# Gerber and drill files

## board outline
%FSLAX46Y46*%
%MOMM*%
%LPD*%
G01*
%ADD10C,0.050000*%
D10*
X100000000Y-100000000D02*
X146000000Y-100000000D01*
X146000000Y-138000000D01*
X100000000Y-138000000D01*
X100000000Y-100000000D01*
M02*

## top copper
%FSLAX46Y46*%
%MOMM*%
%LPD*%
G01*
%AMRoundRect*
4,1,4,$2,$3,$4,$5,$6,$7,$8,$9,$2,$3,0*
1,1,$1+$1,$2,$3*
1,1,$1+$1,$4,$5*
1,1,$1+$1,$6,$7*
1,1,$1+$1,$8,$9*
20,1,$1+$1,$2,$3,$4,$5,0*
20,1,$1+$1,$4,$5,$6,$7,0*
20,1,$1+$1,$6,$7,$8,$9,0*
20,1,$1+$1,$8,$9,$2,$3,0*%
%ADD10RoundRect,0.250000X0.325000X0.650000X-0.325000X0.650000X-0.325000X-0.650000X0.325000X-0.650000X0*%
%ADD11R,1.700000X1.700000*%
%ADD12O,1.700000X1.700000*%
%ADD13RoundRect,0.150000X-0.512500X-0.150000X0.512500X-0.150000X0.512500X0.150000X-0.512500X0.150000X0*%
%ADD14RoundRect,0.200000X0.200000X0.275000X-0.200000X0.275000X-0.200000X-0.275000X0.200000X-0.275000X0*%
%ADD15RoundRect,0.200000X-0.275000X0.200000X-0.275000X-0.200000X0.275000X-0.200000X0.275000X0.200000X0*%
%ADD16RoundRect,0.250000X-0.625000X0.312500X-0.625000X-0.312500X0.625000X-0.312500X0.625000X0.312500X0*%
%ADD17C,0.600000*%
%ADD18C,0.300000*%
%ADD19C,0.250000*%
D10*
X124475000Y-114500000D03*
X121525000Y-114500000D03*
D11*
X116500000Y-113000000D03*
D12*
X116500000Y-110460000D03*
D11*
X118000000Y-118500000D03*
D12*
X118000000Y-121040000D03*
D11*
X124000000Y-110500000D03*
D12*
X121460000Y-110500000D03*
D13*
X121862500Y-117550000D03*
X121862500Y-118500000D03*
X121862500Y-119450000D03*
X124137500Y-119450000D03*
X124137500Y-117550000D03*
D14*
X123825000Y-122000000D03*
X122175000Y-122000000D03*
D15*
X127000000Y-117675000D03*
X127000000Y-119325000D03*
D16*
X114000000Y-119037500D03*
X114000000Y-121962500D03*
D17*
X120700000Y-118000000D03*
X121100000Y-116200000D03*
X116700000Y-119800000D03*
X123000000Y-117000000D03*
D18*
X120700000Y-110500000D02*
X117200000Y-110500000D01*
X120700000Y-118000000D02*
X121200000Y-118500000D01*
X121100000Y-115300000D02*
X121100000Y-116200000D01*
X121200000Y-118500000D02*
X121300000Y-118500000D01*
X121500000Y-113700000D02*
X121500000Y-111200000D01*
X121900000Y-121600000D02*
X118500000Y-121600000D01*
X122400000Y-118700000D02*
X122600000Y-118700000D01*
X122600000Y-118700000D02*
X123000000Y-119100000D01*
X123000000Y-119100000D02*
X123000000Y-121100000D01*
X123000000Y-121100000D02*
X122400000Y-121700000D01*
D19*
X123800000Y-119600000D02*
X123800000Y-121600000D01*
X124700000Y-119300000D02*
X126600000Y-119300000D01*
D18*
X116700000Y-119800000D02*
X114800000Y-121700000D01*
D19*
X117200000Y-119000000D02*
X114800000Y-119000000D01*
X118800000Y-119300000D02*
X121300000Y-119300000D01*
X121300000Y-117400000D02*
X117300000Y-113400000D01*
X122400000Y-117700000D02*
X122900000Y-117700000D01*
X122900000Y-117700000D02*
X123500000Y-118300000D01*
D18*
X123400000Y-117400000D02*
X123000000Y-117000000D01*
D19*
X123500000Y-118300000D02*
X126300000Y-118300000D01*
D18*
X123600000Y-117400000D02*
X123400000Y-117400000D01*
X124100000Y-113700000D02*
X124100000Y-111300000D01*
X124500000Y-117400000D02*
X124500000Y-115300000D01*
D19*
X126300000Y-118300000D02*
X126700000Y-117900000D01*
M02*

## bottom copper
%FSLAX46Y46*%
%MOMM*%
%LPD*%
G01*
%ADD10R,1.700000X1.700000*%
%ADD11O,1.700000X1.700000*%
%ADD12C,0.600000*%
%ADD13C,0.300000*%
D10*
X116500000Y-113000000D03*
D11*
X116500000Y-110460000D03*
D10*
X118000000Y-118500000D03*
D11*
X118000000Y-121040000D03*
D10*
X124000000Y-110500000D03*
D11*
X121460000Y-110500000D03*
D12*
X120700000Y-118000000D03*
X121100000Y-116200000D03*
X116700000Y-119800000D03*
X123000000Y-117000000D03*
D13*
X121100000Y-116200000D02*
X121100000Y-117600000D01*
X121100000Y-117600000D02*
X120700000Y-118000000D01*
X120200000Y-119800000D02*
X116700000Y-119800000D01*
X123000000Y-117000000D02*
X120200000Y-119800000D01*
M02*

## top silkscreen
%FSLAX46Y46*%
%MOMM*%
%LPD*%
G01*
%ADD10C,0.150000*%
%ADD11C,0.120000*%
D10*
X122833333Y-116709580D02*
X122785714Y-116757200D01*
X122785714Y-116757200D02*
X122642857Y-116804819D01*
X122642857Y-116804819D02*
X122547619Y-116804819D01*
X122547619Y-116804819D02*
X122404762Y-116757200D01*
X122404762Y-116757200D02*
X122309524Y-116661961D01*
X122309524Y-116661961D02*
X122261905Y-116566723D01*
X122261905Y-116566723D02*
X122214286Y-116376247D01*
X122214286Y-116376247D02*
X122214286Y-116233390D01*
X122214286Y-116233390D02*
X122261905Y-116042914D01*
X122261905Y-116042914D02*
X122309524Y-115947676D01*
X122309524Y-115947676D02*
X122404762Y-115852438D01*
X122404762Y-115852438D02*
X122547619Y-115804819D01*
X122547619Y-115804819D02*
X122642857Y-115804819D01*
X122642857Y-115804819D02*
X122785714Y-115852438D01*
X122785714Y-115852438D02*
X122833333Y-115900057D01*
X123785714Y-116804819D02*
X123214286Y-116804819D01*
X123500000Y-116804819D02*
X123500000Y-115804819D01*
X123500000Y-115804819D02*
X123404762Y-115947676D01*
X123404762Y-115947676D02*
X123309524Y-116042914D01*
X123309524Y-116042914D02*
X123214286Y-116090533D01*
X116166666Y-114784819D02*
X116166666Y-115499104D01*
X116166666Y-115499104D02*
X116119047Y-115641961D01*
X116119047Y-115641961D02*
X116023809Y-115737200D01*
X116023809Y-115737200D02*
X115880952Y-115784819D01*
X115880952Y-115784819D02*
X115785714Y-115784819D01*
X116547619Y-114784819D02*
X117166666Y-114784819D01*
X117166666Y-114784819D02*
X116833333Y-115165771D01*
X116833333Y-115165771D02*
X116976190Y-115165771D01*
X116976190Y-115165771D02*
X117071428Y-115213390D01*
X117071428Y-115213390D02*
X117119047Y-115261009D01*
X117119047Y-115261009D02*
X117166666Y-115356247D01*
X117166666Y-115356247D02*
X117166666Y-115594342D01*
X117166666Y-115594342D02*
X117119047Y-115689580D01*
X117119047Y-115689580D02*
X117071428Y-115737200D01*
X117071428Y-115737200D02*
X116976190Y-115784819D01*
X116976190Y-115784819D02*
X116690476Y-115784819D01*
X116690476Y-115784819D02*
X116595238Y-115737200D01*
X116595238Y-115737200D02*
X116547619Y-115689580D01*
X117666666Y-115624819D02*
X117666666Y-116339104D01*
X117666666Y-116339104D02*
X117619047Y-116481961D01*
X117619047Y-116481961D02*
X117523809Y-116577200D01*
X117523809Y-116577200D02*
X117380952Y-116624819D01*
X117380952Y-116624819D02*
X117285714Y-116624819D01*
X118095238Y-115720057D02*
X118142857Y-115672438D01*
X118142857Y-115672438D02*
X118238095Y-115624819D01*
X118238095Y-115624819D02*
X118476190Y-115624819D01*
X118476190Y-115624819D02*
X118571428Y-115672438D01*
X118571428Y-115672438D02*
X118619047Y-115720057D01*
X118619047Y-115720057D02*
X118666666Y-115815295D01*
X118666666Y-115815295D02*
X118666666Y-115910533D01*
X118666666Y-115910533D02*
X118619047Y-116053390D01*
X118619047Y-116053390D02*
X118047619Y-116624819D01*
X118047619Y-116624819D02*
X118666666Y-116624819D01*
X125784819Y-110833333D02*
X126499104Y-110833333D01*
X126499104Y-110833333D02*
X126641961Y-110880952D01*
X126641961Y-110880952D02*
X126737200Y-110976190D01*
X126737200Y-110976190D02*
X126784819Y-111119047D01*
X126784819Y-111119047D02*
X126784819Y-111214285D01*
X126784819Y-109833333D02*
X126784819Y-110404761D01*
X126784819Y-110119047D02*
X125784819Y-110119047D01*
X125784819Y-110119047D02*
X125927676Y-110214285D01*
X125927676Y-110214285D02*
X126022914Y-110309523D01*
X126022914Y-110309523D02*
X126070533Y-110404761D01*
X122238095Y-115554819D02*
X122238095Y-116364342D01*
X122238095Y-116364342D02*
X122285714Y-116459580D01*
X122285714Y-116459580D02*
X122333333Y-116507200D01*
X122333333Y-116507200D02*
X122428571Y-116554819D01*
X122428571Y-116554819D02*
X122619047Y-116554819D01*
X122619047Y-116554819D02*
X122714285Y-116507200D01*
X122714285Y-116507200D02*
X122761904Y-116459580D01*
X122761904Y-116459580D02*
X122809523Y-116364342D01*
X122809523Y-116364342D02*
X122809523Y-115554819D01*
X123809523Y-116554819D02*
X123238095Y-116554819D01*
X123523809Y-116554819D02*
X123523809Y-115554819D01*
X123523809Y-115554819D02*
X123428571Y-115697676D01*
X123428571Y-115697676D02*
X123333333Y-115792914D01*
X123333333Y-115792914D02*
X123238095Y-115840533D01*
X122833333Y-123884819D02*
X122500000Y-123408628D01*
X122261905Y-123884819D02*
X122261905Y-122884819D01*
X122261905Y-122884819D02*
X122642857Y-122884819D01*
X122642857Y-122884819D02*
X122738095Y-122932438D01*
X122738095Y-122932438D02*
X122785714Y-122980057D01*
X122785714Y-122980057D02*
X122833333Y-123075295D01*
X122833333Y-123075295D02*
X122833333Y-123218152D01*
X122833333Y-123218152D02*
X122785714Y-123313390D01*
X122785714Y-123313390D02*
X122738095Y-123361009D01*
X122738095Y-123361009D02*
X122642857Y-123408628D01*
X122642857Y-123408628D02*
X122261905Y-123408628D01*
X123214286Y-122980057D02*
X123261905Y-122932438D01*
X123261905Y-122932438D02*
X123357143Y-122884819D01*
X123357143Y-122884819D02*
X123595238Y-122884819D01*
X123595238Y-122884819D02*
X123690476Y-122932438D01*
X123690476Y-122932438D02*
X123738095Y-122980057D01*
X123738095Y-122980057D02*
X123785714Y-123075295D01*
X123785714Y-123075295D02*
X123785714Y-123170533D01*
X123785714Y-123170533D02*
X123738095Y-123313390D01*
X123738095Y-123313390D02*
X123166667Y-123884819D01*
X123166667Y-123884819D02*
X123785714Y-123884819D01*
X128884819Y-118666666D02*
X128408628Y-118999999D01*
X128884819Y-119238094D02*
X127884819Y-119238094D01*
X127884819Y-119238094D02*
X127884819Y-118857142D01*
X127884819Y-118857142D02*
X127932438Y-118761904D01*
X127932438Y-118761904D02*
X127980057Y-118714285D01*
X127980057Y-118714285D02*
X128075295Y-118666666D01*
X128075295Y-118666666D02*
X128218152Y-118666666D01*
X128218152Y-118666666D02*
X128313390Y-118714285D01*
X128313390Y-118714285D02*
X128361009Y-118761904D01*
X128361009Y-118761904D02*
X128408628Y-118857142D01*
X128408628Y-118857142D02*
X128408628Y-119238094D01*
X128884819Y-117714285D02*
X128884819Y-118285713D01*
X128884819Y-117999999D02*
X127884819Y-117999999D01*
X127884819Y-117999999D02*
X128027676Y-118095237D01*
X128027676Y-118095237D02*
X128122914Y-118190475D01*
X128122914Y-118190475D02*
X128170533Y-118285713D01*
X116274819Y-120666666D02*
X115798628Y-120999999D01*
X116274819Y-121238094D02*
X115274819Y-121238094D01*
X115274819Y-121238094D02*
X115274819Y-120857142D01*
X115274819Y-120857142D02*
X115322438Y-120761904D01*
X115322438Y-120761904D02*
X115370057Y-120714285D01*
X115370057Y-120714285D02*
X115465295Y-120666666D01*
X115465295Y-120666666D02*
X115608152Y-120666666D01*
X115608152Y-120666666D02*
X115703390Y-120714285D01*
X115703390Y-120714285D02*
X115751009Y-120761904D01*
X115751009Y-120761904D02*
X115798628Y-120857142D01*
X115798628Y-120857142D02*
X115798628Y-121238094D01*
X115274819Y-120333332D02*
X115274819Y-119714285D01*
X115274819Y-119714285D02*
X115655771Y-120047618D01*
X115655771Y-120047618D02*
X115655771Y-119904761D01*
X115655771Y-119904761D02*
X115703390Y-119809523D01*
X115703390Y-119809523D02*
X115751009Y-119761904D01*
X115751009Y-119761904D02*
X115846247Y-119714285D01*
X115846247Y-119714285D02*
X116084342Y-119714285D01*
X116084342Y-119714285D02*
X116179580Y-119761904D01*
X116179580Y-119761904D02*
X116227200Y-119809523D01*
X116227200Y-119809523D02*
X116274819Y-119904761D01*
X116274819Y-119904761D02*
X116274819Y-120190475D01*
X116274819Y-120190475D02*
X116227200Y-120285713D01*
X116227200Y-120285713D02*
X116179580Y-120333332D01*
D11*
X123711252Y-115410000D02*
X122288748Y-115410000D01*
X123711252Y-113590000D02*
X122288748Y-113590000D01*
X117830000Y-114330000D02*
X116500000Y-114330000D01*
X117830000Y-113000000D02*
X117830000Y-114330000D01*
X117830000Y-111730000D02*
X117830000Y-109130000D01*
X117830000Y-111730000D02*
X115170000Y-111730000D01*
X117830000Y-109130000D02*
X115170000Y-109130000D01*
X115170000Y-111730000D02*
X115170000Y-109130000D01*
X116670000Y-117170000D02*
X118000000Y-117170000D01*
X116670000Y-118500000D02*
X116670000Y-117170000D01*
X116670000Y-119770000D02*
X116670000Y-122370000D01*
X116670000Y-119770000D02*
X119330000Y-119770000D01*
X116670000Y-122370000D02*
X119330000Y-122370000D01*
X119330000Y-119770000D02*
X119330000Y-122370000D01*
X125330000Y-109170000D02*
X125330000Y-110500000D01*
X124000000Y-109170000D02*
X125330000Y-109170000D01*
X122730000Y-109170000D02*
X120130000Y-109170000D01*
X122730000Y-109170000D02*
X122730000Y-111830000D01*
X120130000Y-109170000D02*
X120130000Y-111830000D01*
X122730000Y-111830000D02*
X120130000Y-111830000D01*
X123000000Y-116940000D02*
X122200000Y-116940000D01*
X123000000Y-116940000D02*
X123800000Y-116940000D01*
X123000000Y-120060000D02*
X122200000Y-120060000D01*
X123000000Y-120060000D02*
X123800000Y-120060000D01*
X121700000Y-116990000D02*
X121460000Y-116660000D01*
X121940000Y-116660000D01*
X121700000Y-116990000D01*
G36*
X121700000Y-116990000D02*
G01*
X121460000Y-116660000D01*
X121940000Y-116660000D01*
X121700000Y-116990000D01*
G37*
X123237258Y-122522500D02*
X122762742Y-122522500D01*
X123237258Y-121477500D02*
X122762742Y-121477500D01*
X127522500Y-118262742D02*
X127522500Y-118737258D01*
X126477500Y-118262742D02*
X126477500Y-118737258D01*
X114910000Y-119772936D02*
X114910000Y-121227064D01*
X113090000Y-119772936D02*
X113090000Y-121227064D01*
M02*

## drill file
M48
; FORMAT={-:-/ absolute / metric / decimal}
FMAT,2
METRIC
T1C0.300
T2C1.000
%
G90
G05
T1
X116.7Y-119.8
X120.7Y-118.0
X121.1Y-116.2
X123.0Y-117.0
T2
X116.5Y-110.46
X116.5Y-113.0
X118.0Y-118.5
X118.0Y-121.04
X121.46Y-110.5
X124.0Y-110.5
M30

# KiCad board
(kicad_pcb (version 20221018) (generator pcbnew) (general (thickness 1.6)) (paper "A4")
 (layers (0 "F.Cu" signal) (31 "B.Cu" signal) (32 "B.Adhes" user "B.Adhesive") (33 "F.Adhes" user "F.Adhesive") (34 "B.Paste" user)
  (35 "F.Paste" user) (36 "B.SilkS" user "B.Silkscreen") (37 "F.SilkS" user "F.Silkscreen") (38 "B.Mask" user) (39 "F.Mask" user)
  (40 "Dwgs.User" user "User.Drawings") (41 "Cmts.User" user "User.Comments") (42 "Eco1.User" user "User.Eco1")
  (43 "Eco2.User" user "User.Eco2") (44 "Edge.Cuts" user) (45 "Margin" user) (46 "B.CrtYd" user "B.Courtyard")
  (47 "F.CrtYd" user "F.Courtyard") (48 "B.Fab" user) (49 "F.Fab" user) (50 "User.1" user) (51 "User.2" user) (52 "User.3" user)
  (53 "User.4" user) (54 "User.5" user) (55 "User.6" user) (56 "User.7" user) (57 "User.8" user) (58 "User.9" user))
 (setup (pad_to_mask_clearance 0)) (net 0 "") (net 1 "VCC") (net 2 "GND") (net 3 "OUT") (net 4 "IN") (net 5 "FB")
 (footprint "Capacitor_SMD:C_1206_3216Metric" (layer "F.Cu") (at 123 114.5 180)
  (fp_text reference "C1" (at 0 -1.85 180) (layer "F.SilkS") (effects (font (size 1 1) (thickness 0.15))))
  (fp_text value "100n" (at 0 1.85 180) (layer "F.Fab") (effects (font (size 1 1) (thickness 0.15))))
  (fp_line (start -0.711252 -0.91) (end 0.711252 -0.91) (stroke (width 0.12) (type solid)) (layer "F.SilkS"))
  (fp_line (start -0.711252 0.91) (end 0.711252 0.91) (stroke (width 0.12) (type solid)) (layer "F.SilkS"))
  (pad "1" smd roundrect (at -1.475 0 180) (size 1.15 1.8) (layers "F.Cu" "F.Paste" "F.Mask") (roundrect_rratio 0.217391) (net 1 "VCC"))
  (pad "2" smd roundrect (at 1.475 0 180) (size 1.15 1.8) (layers "F.Cu" "F.Paste" "F.Mask") (roundrect_rratio 0.217391) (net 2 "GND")))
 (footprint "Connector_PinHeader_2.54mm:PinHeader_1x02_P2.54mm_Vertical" (layer "F.Cu") (at 116.5 113 180)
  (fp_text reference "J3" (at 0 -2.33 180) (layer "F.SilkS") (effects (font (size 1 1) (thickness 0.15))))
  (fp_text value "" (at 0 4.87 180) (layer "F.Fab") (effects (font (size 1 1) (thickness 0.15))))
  (fp_line (start -1.33 -1.33) (end 0 -1.33) (stroke (width 0.12) (type solid)) (layer "F.SilkS"))
  (fp_line (start -1.33 0) (end -1.33 -1.33) (stroke (width 0.12) (type solid)) (layer "F.SilkS"))
  (fp_line (start -1.33 1.27) (end -1.33 3.87) (stroke (width 0.12) (type solid)) (layer "F.SilkS"))
  (fp_line (start -1.33 1.27) (end 1.33 1.27) (stroke (width 0.12) (type solid)) (layer "F.SilkS"))
  (fp_line (start -1.33 3.87) (end 1.33 3.87) (stroke (width 0.12) (type solid)) (layer "F.SilkS"))
  (fp_line (start 1.33 1.27) (end 1.33 3.87) (stroke (width 0.12) (type solid)) (layer "F.SilkS"))
  (pad "1" thru_hole rect (at 0 0 180) (size 1.7 1.7) (drill 1) (layers "*.Cu" "*.Mask") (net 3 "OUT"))
  (pad "2" thru_hole oval (at 0 2.54 180) (size 1.7 1.7) (drill 1) (layers "*.Cu" "*.Mask") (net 2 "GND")))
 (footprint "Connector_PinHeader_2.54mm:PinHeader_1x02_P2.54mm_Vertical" (layer "F.Cu") (at 118 118.5)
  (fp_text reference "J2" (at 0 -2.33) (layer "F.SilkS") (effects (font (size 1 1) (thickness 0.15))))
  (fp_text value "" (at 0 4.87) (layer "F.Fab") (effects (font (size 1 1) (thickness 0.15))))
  (fp_line (start -1.33 -1.33) (end 0 -1.33) (stroke (width 0.12) (type solid)) (layer "F.SilkS"))
  (fp_line (start -1.33 0) (end -1.33 -1.33) (stroke (width 0.12) (type solid)) (layer "F.SilkS"))
  (fp_line (start -1.33 1.27) (end -1.33 3.87) (stroke (width 0.12) (type solid)) (layer "F.SilkS"))
  (fp_line (start -1.33 1.27) (end 1.33 1.27) (stroke (width 0.12) (type solid)) (layer "F.SilkS"))
  (fp_line (start -1.33 3.87) (end 1.33 3.87) (stroke (width 0.12) (type solid)) (layer "F.SilkS"))
  (fp_line (start 1.33 1.27) (end 1.33 3.87) (stroke (width 0.12) (type solid)) (layer "F.SilkS"))
  (pad "1" thru_hole rect (at 0 0) (size 1.7 1.7) (drill 1) (layers "*.Cu" "*.Mask") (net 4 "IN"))
  (pad "2" thru_hole oval (at 0 2.54) (size 1.7 1.7) (drill 1) (layers "*.Cu" "*.Mask") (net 2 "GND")))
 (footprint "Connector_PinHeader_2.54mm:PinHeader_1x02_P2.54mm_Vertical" (layer "F.Cu") (at 124 110.5 -90)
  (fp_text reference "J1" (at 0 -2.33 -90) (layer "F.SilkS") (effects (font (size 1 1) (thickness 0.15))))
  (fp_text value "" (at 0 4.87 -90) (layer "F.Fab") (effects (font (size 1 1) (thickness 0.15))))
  (fp_line (start -1.33 -1.33) (end 0 -1.33) (stroke (width 0.12) (type solid)) (layer "F.SilkS"))
  (fp_line (start -1.33 0) (end -1.33 -1.33) (stroke (width 0.12) (type solid)) (layer "F.SilkS"))
  (fp_line (start -1.33 1.27) (end -1.33 3.87) (stroke (width 0.12) (type solid)) (layer "F.SilkS"))
  (fp_line (start -1.33 1.27) (end 1.33 1.27) (stroke (width 0.12) (type solid)) (layer "F.SilkS"))
  (fp_line (start -1.33 3.87) (end 1.33 3.87) (stroke (width 0.12) (type solid)) (layer "F.SilkS"))
  (fp_line (start 1.33 1.27) (end 1.33 3.87) (stroke (width 0.12) (type solid)) (layer "F.SilkS"))
  (pad "1" thru_hole rect (at 0 0 270) (size 1.7 1.7) (drill 1) (layers "*.Cu" "*.Mask") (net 1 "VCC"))
  (pad "2" thru_hole oval (at 0 2.54 270) (size 1.7 1.7) (drill 1) (layers "*.Cu" "*.Mask") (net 2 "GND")))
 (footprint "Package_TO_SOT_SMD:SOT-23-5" (layer "F.Cu") (at 123 118.5)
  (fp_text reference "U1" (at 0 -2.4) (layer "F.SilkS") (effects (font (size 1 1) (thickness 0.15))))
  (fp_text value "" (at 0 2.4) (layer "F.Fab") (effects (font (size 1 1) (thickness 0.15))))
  (fp_line (start 0 -1.56) (end -0.8 -1.56) (stroke (width 0.12) (type solid)) (layer "F.SilkS"))
  (fp_line (start 0 -1.56) (end 0.8 -1.56) (stroke (width 0.12) (type solid)) (layer "F.SilkS"))
  (fp_line (start 0 1.56) (end -0.8 1.56) (stroke (width 0.12) (type solid)) (layer "F.SilkS"))
  (fp_line (start 0 1.56) (end 0.8 1.56) (stroke (width 0.12) (type solid)) (layer "F.SilkS"))
  (fp_poly
   (pts (xy -1.3 -1.51) (xy -1.54 -1.84) (xy -1.06 -1.84) (xy -1.3 -1.51)) (stroke (width 0.12) (type solid)) (fill solid) (layer "F.SilkS"))
  (pad "1" smd roundrect (at -1.1375 -0.95) (size 1.325 0.6) (layers "F.Cu" "F.Paste" "F.Mask") (roundrect_rratio 0.25) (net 3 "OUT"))
  (pad "2" smd roundrect (at -1.1375 0) (size 1.325 0.6) (layers "F.Cu" "F.Paste" "F.Mask") (roundrect_rratio 0.25) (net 2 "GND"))
  (pad "3" smd roundrect (at -1.1375 0.95) (size 1.325 0.6) (layers "F.Cu" "F.Paste" "F.Mask") (roundrect_rratio 0.25) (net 4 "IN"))
  (pad "4" smd roundrect (at 1.1375 0.95) (size 1.325 0.6) (layers "F.Cu" "F.Paste" "F.Mask") (roundrect_rratio 0.25) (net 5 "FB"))
  (pad "5" smd roundrect (at 1.1375 -0.95) (size 1.325 0.6) (layers "F.Cu" "F.Paste" "F.Mask") (roundrect_rratio 0.25) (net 1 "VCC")))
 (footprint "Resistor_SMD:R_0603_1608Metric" (layer "F.Cu") (at 123 122 180)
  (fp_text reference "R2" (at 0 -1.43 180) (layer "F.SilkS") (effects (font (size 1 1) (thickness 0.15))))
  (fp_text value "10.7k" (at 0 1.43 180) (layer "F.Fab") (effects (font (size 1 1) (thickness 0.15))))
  (fp_line (start -0.237258 -0.5225) (end 0.237258 -0.5225) (stroke (width 0.12) (type solid)) (layer "F.SilkS"))
  (fp_line (start -0.237258 0.5225) (end 0.237258 0.5225) (stroke (width 0.12) (type solid)) (layer "F.SilkS"))
  (pad "1" smd roundrect (at -0.825 0 180) (size 0.8 0.95) (layers "F.Cu" "F.Paste" "F.Mask") (roundrect_rratio 0.25) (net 5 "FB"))
  (pad "2" smd roundrect (at 0.825 0 180) (size 0.8 0.95) (layers "F.Cu" "F.Paste" "F.Mask") (roundrect_rratio 0.25) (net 2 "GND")))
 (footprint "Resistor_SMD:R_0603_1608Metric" (layer "F.Cu") (at 127 118.5 -90)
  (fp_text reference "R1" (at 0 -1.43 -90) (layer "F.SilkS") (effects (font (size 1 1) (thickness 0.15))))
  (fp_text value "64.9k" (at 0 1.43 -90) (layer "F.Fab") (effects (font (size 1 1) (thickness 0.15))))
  (fp_line (start -0.237258 -0.5225) (end 0.237258 -0.5225) (stroke (width 0.12) (type solid)) (layer "F.SilkS"))
  (fp_line (start -0.237258 0.5225) (end 0.237258 0.5225) (stroke (width 0.12) (type solid)) (layer "F.SilkS"))
  (pad "1" smd roundrect (at -0.825 0 270) (size 0.8 0.95) (layers "F.Cu" "F.Paste" "F.Mask") (roundrect_rratio 0.25) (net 3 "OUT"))
  (pad "2" smd roundrect (at 0.825 0 270) (size 0.8 0.95) (layers "F.Cu" "F.Paste" "F.Mask") (roundrect_rratio 0.25) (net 5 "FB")))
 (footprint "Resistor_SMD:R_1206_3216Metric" (layer "F.Cu") (at 114 120.5 -90)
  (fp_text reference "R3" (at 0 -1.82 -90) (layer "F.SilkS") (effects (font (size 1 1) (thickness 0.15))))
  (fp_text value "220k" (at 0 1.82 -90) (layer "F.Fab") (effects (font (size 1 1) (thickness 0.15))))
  (fp_line (start -0.727064 -0.91) (end 0.727064 -0.91) (stroke (width 0.12) (type solid)) (layer "F.SilkS"))
  (fp_line (start -0.727064 0.91) (end 0.727064 0.91) (stroke (width 0.12) (type solid)) (layer "F.SilkS"))
  (pad "1" smd roundrect (at -1.4625 0 270) (size 1.125 1.75) (layers "F.Cu" "F.Paste" "F.Mask") (roundrect_rratio 0.222222) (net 4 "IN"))
  (pad "2" smd roundrect (at 1.4625 0 270) (size 1.125 1.75) (layers "F.Cu" "F.Paste" "F.Mask") (roundrect_rratio 0.222222) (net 1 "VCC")))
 (gr_rect (start 100 100) (end 146 138) (stroke (width 0.05) (type default)) (fill none) (layer "Edge.Cuts"))
 (segment (start 120.7 110.5) (end 117.2 110.5) (width 0.3) (layer "F.Cu") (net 2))
 (segment (start 120.7 118) (end 121.2 118.5) (width 0.3) (layer "F.Cu") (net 2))
 (segment (start 121.1 115.3) (end 121.1 116.2) (width 0.3) (layer "F.Cu") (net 2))
 (segment (start 121.2 118.5) (end 121.3 118.5) (width 0.3) (layer "F.Cu") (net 2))
 (segment (start 121.5 113.7) (end 121.5 111.2) (width 0.3) (layer "F.Cu") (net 2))
 (segment (start 121.9 121.6) (end 118.5 121.6) (width 0.3) (layer "F.Cu") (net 2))
 (segment (start 122.4 118.7) (end 122.6 118.7) (width 0.3) (layer "F.Cu") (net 2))
 (segment (start 122.6 118.7) (end 123 119.1) (width 0.3) (layer "F.Cu") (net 2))
 (segment (start 123 119.1) (end 123 121.1) (width 0.3) (layer "F.Cu") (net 2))
 (segment (start 123 121.1) (end 122.4 121.7) (width 0.3) (layer "F.Cu") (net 2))
 (segment (start 123.8 119.6) (end 123.8 121.6) (width 0.25) (layer "F.Cu") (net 5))
 (segment (start 124.7 119.3) (end 126.6 119.3) (width 0.25) (layer "F.Cu") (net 5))
 (via (at 120.7 118) (size 0.6) (drill 0.3) (layers "F.Cu" "B.Cu") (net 2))
 (via (at 121.1 116.2) (size 0.6) (drill 0.3) (layers "F.Cu" "B.Cu") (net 2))
 (segment (start 116.7 119.8) (end 114.8 121.7) (width 0.3) (layer "F.Cu") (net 1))
 (segment (start 117.2 119) (end 114.8 119) (width 0.25) (layer "F.Cu") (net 4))
 (segment (start 118.8 119.3) (end 121.3 119.3) (width 0.25) (layer "F.Cu") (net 4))
 (segment (start 121.1 116.2) (end 121.1 117.6) (width 0.3) (layer "B.Cu") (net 2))
 (segment (start 121.1 117.6) (end 120.7 118) (width 0.3) (layer "B.Cu") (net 2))
 (segment (start 121.3 117.4) (end 117.3 113.4) (width 0.25) (layer "F.Cu") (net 3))
 (segment (start 122.4 117.7) (end 122.9 117.7) (width 0.25) (layer "F.Cu") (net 3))
 (segment (start 122.9 117.7) (end 123.5 118.3) (width 0.25) (layer "F.Cu") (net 3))
 (segment (start 123.4 117.4) (end 123 117) (width 0.3) (layer "F.Cu") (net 1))
 (segment (start 123.5 118.3) (end 126.3 118.3) (width 0.25) (layer "F.Cu") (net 3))
 (segment (start 123.6 117.4) (end 123.4 117.4) (width 0.3) (layer "F.Cu") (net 1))
 (segment (start 124.1 113.7) (end 124.1 111.3) (width 0.3) (layer "F.Cu") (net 1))
 (segment (start 124.5 117.4) (end 124.5 115.3) (width 0.3) (layer "F.Cu") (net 1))
 (segment (start 126.3 118.3) (end 126.7 117.9) (width 0.25) (layer "F.Cu") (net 3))
 (via (at 116.7 119.8) (size 0.6) (drill 0.3) (layers "F.Cu" "B.Cu") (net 1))
 (via (at 123 117) (size 0.6) (drill 0.3) (layers "F.Cu" "B.Cu") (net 1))
 (segment (start 120.2 119.8) (end 116.7 119.8) (width 0.3) (layer "B.Cu") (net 1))
 (segment (start 123 117) (end 120.2 119.8) (width 0.3) (layer "B.Cu") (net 1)))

